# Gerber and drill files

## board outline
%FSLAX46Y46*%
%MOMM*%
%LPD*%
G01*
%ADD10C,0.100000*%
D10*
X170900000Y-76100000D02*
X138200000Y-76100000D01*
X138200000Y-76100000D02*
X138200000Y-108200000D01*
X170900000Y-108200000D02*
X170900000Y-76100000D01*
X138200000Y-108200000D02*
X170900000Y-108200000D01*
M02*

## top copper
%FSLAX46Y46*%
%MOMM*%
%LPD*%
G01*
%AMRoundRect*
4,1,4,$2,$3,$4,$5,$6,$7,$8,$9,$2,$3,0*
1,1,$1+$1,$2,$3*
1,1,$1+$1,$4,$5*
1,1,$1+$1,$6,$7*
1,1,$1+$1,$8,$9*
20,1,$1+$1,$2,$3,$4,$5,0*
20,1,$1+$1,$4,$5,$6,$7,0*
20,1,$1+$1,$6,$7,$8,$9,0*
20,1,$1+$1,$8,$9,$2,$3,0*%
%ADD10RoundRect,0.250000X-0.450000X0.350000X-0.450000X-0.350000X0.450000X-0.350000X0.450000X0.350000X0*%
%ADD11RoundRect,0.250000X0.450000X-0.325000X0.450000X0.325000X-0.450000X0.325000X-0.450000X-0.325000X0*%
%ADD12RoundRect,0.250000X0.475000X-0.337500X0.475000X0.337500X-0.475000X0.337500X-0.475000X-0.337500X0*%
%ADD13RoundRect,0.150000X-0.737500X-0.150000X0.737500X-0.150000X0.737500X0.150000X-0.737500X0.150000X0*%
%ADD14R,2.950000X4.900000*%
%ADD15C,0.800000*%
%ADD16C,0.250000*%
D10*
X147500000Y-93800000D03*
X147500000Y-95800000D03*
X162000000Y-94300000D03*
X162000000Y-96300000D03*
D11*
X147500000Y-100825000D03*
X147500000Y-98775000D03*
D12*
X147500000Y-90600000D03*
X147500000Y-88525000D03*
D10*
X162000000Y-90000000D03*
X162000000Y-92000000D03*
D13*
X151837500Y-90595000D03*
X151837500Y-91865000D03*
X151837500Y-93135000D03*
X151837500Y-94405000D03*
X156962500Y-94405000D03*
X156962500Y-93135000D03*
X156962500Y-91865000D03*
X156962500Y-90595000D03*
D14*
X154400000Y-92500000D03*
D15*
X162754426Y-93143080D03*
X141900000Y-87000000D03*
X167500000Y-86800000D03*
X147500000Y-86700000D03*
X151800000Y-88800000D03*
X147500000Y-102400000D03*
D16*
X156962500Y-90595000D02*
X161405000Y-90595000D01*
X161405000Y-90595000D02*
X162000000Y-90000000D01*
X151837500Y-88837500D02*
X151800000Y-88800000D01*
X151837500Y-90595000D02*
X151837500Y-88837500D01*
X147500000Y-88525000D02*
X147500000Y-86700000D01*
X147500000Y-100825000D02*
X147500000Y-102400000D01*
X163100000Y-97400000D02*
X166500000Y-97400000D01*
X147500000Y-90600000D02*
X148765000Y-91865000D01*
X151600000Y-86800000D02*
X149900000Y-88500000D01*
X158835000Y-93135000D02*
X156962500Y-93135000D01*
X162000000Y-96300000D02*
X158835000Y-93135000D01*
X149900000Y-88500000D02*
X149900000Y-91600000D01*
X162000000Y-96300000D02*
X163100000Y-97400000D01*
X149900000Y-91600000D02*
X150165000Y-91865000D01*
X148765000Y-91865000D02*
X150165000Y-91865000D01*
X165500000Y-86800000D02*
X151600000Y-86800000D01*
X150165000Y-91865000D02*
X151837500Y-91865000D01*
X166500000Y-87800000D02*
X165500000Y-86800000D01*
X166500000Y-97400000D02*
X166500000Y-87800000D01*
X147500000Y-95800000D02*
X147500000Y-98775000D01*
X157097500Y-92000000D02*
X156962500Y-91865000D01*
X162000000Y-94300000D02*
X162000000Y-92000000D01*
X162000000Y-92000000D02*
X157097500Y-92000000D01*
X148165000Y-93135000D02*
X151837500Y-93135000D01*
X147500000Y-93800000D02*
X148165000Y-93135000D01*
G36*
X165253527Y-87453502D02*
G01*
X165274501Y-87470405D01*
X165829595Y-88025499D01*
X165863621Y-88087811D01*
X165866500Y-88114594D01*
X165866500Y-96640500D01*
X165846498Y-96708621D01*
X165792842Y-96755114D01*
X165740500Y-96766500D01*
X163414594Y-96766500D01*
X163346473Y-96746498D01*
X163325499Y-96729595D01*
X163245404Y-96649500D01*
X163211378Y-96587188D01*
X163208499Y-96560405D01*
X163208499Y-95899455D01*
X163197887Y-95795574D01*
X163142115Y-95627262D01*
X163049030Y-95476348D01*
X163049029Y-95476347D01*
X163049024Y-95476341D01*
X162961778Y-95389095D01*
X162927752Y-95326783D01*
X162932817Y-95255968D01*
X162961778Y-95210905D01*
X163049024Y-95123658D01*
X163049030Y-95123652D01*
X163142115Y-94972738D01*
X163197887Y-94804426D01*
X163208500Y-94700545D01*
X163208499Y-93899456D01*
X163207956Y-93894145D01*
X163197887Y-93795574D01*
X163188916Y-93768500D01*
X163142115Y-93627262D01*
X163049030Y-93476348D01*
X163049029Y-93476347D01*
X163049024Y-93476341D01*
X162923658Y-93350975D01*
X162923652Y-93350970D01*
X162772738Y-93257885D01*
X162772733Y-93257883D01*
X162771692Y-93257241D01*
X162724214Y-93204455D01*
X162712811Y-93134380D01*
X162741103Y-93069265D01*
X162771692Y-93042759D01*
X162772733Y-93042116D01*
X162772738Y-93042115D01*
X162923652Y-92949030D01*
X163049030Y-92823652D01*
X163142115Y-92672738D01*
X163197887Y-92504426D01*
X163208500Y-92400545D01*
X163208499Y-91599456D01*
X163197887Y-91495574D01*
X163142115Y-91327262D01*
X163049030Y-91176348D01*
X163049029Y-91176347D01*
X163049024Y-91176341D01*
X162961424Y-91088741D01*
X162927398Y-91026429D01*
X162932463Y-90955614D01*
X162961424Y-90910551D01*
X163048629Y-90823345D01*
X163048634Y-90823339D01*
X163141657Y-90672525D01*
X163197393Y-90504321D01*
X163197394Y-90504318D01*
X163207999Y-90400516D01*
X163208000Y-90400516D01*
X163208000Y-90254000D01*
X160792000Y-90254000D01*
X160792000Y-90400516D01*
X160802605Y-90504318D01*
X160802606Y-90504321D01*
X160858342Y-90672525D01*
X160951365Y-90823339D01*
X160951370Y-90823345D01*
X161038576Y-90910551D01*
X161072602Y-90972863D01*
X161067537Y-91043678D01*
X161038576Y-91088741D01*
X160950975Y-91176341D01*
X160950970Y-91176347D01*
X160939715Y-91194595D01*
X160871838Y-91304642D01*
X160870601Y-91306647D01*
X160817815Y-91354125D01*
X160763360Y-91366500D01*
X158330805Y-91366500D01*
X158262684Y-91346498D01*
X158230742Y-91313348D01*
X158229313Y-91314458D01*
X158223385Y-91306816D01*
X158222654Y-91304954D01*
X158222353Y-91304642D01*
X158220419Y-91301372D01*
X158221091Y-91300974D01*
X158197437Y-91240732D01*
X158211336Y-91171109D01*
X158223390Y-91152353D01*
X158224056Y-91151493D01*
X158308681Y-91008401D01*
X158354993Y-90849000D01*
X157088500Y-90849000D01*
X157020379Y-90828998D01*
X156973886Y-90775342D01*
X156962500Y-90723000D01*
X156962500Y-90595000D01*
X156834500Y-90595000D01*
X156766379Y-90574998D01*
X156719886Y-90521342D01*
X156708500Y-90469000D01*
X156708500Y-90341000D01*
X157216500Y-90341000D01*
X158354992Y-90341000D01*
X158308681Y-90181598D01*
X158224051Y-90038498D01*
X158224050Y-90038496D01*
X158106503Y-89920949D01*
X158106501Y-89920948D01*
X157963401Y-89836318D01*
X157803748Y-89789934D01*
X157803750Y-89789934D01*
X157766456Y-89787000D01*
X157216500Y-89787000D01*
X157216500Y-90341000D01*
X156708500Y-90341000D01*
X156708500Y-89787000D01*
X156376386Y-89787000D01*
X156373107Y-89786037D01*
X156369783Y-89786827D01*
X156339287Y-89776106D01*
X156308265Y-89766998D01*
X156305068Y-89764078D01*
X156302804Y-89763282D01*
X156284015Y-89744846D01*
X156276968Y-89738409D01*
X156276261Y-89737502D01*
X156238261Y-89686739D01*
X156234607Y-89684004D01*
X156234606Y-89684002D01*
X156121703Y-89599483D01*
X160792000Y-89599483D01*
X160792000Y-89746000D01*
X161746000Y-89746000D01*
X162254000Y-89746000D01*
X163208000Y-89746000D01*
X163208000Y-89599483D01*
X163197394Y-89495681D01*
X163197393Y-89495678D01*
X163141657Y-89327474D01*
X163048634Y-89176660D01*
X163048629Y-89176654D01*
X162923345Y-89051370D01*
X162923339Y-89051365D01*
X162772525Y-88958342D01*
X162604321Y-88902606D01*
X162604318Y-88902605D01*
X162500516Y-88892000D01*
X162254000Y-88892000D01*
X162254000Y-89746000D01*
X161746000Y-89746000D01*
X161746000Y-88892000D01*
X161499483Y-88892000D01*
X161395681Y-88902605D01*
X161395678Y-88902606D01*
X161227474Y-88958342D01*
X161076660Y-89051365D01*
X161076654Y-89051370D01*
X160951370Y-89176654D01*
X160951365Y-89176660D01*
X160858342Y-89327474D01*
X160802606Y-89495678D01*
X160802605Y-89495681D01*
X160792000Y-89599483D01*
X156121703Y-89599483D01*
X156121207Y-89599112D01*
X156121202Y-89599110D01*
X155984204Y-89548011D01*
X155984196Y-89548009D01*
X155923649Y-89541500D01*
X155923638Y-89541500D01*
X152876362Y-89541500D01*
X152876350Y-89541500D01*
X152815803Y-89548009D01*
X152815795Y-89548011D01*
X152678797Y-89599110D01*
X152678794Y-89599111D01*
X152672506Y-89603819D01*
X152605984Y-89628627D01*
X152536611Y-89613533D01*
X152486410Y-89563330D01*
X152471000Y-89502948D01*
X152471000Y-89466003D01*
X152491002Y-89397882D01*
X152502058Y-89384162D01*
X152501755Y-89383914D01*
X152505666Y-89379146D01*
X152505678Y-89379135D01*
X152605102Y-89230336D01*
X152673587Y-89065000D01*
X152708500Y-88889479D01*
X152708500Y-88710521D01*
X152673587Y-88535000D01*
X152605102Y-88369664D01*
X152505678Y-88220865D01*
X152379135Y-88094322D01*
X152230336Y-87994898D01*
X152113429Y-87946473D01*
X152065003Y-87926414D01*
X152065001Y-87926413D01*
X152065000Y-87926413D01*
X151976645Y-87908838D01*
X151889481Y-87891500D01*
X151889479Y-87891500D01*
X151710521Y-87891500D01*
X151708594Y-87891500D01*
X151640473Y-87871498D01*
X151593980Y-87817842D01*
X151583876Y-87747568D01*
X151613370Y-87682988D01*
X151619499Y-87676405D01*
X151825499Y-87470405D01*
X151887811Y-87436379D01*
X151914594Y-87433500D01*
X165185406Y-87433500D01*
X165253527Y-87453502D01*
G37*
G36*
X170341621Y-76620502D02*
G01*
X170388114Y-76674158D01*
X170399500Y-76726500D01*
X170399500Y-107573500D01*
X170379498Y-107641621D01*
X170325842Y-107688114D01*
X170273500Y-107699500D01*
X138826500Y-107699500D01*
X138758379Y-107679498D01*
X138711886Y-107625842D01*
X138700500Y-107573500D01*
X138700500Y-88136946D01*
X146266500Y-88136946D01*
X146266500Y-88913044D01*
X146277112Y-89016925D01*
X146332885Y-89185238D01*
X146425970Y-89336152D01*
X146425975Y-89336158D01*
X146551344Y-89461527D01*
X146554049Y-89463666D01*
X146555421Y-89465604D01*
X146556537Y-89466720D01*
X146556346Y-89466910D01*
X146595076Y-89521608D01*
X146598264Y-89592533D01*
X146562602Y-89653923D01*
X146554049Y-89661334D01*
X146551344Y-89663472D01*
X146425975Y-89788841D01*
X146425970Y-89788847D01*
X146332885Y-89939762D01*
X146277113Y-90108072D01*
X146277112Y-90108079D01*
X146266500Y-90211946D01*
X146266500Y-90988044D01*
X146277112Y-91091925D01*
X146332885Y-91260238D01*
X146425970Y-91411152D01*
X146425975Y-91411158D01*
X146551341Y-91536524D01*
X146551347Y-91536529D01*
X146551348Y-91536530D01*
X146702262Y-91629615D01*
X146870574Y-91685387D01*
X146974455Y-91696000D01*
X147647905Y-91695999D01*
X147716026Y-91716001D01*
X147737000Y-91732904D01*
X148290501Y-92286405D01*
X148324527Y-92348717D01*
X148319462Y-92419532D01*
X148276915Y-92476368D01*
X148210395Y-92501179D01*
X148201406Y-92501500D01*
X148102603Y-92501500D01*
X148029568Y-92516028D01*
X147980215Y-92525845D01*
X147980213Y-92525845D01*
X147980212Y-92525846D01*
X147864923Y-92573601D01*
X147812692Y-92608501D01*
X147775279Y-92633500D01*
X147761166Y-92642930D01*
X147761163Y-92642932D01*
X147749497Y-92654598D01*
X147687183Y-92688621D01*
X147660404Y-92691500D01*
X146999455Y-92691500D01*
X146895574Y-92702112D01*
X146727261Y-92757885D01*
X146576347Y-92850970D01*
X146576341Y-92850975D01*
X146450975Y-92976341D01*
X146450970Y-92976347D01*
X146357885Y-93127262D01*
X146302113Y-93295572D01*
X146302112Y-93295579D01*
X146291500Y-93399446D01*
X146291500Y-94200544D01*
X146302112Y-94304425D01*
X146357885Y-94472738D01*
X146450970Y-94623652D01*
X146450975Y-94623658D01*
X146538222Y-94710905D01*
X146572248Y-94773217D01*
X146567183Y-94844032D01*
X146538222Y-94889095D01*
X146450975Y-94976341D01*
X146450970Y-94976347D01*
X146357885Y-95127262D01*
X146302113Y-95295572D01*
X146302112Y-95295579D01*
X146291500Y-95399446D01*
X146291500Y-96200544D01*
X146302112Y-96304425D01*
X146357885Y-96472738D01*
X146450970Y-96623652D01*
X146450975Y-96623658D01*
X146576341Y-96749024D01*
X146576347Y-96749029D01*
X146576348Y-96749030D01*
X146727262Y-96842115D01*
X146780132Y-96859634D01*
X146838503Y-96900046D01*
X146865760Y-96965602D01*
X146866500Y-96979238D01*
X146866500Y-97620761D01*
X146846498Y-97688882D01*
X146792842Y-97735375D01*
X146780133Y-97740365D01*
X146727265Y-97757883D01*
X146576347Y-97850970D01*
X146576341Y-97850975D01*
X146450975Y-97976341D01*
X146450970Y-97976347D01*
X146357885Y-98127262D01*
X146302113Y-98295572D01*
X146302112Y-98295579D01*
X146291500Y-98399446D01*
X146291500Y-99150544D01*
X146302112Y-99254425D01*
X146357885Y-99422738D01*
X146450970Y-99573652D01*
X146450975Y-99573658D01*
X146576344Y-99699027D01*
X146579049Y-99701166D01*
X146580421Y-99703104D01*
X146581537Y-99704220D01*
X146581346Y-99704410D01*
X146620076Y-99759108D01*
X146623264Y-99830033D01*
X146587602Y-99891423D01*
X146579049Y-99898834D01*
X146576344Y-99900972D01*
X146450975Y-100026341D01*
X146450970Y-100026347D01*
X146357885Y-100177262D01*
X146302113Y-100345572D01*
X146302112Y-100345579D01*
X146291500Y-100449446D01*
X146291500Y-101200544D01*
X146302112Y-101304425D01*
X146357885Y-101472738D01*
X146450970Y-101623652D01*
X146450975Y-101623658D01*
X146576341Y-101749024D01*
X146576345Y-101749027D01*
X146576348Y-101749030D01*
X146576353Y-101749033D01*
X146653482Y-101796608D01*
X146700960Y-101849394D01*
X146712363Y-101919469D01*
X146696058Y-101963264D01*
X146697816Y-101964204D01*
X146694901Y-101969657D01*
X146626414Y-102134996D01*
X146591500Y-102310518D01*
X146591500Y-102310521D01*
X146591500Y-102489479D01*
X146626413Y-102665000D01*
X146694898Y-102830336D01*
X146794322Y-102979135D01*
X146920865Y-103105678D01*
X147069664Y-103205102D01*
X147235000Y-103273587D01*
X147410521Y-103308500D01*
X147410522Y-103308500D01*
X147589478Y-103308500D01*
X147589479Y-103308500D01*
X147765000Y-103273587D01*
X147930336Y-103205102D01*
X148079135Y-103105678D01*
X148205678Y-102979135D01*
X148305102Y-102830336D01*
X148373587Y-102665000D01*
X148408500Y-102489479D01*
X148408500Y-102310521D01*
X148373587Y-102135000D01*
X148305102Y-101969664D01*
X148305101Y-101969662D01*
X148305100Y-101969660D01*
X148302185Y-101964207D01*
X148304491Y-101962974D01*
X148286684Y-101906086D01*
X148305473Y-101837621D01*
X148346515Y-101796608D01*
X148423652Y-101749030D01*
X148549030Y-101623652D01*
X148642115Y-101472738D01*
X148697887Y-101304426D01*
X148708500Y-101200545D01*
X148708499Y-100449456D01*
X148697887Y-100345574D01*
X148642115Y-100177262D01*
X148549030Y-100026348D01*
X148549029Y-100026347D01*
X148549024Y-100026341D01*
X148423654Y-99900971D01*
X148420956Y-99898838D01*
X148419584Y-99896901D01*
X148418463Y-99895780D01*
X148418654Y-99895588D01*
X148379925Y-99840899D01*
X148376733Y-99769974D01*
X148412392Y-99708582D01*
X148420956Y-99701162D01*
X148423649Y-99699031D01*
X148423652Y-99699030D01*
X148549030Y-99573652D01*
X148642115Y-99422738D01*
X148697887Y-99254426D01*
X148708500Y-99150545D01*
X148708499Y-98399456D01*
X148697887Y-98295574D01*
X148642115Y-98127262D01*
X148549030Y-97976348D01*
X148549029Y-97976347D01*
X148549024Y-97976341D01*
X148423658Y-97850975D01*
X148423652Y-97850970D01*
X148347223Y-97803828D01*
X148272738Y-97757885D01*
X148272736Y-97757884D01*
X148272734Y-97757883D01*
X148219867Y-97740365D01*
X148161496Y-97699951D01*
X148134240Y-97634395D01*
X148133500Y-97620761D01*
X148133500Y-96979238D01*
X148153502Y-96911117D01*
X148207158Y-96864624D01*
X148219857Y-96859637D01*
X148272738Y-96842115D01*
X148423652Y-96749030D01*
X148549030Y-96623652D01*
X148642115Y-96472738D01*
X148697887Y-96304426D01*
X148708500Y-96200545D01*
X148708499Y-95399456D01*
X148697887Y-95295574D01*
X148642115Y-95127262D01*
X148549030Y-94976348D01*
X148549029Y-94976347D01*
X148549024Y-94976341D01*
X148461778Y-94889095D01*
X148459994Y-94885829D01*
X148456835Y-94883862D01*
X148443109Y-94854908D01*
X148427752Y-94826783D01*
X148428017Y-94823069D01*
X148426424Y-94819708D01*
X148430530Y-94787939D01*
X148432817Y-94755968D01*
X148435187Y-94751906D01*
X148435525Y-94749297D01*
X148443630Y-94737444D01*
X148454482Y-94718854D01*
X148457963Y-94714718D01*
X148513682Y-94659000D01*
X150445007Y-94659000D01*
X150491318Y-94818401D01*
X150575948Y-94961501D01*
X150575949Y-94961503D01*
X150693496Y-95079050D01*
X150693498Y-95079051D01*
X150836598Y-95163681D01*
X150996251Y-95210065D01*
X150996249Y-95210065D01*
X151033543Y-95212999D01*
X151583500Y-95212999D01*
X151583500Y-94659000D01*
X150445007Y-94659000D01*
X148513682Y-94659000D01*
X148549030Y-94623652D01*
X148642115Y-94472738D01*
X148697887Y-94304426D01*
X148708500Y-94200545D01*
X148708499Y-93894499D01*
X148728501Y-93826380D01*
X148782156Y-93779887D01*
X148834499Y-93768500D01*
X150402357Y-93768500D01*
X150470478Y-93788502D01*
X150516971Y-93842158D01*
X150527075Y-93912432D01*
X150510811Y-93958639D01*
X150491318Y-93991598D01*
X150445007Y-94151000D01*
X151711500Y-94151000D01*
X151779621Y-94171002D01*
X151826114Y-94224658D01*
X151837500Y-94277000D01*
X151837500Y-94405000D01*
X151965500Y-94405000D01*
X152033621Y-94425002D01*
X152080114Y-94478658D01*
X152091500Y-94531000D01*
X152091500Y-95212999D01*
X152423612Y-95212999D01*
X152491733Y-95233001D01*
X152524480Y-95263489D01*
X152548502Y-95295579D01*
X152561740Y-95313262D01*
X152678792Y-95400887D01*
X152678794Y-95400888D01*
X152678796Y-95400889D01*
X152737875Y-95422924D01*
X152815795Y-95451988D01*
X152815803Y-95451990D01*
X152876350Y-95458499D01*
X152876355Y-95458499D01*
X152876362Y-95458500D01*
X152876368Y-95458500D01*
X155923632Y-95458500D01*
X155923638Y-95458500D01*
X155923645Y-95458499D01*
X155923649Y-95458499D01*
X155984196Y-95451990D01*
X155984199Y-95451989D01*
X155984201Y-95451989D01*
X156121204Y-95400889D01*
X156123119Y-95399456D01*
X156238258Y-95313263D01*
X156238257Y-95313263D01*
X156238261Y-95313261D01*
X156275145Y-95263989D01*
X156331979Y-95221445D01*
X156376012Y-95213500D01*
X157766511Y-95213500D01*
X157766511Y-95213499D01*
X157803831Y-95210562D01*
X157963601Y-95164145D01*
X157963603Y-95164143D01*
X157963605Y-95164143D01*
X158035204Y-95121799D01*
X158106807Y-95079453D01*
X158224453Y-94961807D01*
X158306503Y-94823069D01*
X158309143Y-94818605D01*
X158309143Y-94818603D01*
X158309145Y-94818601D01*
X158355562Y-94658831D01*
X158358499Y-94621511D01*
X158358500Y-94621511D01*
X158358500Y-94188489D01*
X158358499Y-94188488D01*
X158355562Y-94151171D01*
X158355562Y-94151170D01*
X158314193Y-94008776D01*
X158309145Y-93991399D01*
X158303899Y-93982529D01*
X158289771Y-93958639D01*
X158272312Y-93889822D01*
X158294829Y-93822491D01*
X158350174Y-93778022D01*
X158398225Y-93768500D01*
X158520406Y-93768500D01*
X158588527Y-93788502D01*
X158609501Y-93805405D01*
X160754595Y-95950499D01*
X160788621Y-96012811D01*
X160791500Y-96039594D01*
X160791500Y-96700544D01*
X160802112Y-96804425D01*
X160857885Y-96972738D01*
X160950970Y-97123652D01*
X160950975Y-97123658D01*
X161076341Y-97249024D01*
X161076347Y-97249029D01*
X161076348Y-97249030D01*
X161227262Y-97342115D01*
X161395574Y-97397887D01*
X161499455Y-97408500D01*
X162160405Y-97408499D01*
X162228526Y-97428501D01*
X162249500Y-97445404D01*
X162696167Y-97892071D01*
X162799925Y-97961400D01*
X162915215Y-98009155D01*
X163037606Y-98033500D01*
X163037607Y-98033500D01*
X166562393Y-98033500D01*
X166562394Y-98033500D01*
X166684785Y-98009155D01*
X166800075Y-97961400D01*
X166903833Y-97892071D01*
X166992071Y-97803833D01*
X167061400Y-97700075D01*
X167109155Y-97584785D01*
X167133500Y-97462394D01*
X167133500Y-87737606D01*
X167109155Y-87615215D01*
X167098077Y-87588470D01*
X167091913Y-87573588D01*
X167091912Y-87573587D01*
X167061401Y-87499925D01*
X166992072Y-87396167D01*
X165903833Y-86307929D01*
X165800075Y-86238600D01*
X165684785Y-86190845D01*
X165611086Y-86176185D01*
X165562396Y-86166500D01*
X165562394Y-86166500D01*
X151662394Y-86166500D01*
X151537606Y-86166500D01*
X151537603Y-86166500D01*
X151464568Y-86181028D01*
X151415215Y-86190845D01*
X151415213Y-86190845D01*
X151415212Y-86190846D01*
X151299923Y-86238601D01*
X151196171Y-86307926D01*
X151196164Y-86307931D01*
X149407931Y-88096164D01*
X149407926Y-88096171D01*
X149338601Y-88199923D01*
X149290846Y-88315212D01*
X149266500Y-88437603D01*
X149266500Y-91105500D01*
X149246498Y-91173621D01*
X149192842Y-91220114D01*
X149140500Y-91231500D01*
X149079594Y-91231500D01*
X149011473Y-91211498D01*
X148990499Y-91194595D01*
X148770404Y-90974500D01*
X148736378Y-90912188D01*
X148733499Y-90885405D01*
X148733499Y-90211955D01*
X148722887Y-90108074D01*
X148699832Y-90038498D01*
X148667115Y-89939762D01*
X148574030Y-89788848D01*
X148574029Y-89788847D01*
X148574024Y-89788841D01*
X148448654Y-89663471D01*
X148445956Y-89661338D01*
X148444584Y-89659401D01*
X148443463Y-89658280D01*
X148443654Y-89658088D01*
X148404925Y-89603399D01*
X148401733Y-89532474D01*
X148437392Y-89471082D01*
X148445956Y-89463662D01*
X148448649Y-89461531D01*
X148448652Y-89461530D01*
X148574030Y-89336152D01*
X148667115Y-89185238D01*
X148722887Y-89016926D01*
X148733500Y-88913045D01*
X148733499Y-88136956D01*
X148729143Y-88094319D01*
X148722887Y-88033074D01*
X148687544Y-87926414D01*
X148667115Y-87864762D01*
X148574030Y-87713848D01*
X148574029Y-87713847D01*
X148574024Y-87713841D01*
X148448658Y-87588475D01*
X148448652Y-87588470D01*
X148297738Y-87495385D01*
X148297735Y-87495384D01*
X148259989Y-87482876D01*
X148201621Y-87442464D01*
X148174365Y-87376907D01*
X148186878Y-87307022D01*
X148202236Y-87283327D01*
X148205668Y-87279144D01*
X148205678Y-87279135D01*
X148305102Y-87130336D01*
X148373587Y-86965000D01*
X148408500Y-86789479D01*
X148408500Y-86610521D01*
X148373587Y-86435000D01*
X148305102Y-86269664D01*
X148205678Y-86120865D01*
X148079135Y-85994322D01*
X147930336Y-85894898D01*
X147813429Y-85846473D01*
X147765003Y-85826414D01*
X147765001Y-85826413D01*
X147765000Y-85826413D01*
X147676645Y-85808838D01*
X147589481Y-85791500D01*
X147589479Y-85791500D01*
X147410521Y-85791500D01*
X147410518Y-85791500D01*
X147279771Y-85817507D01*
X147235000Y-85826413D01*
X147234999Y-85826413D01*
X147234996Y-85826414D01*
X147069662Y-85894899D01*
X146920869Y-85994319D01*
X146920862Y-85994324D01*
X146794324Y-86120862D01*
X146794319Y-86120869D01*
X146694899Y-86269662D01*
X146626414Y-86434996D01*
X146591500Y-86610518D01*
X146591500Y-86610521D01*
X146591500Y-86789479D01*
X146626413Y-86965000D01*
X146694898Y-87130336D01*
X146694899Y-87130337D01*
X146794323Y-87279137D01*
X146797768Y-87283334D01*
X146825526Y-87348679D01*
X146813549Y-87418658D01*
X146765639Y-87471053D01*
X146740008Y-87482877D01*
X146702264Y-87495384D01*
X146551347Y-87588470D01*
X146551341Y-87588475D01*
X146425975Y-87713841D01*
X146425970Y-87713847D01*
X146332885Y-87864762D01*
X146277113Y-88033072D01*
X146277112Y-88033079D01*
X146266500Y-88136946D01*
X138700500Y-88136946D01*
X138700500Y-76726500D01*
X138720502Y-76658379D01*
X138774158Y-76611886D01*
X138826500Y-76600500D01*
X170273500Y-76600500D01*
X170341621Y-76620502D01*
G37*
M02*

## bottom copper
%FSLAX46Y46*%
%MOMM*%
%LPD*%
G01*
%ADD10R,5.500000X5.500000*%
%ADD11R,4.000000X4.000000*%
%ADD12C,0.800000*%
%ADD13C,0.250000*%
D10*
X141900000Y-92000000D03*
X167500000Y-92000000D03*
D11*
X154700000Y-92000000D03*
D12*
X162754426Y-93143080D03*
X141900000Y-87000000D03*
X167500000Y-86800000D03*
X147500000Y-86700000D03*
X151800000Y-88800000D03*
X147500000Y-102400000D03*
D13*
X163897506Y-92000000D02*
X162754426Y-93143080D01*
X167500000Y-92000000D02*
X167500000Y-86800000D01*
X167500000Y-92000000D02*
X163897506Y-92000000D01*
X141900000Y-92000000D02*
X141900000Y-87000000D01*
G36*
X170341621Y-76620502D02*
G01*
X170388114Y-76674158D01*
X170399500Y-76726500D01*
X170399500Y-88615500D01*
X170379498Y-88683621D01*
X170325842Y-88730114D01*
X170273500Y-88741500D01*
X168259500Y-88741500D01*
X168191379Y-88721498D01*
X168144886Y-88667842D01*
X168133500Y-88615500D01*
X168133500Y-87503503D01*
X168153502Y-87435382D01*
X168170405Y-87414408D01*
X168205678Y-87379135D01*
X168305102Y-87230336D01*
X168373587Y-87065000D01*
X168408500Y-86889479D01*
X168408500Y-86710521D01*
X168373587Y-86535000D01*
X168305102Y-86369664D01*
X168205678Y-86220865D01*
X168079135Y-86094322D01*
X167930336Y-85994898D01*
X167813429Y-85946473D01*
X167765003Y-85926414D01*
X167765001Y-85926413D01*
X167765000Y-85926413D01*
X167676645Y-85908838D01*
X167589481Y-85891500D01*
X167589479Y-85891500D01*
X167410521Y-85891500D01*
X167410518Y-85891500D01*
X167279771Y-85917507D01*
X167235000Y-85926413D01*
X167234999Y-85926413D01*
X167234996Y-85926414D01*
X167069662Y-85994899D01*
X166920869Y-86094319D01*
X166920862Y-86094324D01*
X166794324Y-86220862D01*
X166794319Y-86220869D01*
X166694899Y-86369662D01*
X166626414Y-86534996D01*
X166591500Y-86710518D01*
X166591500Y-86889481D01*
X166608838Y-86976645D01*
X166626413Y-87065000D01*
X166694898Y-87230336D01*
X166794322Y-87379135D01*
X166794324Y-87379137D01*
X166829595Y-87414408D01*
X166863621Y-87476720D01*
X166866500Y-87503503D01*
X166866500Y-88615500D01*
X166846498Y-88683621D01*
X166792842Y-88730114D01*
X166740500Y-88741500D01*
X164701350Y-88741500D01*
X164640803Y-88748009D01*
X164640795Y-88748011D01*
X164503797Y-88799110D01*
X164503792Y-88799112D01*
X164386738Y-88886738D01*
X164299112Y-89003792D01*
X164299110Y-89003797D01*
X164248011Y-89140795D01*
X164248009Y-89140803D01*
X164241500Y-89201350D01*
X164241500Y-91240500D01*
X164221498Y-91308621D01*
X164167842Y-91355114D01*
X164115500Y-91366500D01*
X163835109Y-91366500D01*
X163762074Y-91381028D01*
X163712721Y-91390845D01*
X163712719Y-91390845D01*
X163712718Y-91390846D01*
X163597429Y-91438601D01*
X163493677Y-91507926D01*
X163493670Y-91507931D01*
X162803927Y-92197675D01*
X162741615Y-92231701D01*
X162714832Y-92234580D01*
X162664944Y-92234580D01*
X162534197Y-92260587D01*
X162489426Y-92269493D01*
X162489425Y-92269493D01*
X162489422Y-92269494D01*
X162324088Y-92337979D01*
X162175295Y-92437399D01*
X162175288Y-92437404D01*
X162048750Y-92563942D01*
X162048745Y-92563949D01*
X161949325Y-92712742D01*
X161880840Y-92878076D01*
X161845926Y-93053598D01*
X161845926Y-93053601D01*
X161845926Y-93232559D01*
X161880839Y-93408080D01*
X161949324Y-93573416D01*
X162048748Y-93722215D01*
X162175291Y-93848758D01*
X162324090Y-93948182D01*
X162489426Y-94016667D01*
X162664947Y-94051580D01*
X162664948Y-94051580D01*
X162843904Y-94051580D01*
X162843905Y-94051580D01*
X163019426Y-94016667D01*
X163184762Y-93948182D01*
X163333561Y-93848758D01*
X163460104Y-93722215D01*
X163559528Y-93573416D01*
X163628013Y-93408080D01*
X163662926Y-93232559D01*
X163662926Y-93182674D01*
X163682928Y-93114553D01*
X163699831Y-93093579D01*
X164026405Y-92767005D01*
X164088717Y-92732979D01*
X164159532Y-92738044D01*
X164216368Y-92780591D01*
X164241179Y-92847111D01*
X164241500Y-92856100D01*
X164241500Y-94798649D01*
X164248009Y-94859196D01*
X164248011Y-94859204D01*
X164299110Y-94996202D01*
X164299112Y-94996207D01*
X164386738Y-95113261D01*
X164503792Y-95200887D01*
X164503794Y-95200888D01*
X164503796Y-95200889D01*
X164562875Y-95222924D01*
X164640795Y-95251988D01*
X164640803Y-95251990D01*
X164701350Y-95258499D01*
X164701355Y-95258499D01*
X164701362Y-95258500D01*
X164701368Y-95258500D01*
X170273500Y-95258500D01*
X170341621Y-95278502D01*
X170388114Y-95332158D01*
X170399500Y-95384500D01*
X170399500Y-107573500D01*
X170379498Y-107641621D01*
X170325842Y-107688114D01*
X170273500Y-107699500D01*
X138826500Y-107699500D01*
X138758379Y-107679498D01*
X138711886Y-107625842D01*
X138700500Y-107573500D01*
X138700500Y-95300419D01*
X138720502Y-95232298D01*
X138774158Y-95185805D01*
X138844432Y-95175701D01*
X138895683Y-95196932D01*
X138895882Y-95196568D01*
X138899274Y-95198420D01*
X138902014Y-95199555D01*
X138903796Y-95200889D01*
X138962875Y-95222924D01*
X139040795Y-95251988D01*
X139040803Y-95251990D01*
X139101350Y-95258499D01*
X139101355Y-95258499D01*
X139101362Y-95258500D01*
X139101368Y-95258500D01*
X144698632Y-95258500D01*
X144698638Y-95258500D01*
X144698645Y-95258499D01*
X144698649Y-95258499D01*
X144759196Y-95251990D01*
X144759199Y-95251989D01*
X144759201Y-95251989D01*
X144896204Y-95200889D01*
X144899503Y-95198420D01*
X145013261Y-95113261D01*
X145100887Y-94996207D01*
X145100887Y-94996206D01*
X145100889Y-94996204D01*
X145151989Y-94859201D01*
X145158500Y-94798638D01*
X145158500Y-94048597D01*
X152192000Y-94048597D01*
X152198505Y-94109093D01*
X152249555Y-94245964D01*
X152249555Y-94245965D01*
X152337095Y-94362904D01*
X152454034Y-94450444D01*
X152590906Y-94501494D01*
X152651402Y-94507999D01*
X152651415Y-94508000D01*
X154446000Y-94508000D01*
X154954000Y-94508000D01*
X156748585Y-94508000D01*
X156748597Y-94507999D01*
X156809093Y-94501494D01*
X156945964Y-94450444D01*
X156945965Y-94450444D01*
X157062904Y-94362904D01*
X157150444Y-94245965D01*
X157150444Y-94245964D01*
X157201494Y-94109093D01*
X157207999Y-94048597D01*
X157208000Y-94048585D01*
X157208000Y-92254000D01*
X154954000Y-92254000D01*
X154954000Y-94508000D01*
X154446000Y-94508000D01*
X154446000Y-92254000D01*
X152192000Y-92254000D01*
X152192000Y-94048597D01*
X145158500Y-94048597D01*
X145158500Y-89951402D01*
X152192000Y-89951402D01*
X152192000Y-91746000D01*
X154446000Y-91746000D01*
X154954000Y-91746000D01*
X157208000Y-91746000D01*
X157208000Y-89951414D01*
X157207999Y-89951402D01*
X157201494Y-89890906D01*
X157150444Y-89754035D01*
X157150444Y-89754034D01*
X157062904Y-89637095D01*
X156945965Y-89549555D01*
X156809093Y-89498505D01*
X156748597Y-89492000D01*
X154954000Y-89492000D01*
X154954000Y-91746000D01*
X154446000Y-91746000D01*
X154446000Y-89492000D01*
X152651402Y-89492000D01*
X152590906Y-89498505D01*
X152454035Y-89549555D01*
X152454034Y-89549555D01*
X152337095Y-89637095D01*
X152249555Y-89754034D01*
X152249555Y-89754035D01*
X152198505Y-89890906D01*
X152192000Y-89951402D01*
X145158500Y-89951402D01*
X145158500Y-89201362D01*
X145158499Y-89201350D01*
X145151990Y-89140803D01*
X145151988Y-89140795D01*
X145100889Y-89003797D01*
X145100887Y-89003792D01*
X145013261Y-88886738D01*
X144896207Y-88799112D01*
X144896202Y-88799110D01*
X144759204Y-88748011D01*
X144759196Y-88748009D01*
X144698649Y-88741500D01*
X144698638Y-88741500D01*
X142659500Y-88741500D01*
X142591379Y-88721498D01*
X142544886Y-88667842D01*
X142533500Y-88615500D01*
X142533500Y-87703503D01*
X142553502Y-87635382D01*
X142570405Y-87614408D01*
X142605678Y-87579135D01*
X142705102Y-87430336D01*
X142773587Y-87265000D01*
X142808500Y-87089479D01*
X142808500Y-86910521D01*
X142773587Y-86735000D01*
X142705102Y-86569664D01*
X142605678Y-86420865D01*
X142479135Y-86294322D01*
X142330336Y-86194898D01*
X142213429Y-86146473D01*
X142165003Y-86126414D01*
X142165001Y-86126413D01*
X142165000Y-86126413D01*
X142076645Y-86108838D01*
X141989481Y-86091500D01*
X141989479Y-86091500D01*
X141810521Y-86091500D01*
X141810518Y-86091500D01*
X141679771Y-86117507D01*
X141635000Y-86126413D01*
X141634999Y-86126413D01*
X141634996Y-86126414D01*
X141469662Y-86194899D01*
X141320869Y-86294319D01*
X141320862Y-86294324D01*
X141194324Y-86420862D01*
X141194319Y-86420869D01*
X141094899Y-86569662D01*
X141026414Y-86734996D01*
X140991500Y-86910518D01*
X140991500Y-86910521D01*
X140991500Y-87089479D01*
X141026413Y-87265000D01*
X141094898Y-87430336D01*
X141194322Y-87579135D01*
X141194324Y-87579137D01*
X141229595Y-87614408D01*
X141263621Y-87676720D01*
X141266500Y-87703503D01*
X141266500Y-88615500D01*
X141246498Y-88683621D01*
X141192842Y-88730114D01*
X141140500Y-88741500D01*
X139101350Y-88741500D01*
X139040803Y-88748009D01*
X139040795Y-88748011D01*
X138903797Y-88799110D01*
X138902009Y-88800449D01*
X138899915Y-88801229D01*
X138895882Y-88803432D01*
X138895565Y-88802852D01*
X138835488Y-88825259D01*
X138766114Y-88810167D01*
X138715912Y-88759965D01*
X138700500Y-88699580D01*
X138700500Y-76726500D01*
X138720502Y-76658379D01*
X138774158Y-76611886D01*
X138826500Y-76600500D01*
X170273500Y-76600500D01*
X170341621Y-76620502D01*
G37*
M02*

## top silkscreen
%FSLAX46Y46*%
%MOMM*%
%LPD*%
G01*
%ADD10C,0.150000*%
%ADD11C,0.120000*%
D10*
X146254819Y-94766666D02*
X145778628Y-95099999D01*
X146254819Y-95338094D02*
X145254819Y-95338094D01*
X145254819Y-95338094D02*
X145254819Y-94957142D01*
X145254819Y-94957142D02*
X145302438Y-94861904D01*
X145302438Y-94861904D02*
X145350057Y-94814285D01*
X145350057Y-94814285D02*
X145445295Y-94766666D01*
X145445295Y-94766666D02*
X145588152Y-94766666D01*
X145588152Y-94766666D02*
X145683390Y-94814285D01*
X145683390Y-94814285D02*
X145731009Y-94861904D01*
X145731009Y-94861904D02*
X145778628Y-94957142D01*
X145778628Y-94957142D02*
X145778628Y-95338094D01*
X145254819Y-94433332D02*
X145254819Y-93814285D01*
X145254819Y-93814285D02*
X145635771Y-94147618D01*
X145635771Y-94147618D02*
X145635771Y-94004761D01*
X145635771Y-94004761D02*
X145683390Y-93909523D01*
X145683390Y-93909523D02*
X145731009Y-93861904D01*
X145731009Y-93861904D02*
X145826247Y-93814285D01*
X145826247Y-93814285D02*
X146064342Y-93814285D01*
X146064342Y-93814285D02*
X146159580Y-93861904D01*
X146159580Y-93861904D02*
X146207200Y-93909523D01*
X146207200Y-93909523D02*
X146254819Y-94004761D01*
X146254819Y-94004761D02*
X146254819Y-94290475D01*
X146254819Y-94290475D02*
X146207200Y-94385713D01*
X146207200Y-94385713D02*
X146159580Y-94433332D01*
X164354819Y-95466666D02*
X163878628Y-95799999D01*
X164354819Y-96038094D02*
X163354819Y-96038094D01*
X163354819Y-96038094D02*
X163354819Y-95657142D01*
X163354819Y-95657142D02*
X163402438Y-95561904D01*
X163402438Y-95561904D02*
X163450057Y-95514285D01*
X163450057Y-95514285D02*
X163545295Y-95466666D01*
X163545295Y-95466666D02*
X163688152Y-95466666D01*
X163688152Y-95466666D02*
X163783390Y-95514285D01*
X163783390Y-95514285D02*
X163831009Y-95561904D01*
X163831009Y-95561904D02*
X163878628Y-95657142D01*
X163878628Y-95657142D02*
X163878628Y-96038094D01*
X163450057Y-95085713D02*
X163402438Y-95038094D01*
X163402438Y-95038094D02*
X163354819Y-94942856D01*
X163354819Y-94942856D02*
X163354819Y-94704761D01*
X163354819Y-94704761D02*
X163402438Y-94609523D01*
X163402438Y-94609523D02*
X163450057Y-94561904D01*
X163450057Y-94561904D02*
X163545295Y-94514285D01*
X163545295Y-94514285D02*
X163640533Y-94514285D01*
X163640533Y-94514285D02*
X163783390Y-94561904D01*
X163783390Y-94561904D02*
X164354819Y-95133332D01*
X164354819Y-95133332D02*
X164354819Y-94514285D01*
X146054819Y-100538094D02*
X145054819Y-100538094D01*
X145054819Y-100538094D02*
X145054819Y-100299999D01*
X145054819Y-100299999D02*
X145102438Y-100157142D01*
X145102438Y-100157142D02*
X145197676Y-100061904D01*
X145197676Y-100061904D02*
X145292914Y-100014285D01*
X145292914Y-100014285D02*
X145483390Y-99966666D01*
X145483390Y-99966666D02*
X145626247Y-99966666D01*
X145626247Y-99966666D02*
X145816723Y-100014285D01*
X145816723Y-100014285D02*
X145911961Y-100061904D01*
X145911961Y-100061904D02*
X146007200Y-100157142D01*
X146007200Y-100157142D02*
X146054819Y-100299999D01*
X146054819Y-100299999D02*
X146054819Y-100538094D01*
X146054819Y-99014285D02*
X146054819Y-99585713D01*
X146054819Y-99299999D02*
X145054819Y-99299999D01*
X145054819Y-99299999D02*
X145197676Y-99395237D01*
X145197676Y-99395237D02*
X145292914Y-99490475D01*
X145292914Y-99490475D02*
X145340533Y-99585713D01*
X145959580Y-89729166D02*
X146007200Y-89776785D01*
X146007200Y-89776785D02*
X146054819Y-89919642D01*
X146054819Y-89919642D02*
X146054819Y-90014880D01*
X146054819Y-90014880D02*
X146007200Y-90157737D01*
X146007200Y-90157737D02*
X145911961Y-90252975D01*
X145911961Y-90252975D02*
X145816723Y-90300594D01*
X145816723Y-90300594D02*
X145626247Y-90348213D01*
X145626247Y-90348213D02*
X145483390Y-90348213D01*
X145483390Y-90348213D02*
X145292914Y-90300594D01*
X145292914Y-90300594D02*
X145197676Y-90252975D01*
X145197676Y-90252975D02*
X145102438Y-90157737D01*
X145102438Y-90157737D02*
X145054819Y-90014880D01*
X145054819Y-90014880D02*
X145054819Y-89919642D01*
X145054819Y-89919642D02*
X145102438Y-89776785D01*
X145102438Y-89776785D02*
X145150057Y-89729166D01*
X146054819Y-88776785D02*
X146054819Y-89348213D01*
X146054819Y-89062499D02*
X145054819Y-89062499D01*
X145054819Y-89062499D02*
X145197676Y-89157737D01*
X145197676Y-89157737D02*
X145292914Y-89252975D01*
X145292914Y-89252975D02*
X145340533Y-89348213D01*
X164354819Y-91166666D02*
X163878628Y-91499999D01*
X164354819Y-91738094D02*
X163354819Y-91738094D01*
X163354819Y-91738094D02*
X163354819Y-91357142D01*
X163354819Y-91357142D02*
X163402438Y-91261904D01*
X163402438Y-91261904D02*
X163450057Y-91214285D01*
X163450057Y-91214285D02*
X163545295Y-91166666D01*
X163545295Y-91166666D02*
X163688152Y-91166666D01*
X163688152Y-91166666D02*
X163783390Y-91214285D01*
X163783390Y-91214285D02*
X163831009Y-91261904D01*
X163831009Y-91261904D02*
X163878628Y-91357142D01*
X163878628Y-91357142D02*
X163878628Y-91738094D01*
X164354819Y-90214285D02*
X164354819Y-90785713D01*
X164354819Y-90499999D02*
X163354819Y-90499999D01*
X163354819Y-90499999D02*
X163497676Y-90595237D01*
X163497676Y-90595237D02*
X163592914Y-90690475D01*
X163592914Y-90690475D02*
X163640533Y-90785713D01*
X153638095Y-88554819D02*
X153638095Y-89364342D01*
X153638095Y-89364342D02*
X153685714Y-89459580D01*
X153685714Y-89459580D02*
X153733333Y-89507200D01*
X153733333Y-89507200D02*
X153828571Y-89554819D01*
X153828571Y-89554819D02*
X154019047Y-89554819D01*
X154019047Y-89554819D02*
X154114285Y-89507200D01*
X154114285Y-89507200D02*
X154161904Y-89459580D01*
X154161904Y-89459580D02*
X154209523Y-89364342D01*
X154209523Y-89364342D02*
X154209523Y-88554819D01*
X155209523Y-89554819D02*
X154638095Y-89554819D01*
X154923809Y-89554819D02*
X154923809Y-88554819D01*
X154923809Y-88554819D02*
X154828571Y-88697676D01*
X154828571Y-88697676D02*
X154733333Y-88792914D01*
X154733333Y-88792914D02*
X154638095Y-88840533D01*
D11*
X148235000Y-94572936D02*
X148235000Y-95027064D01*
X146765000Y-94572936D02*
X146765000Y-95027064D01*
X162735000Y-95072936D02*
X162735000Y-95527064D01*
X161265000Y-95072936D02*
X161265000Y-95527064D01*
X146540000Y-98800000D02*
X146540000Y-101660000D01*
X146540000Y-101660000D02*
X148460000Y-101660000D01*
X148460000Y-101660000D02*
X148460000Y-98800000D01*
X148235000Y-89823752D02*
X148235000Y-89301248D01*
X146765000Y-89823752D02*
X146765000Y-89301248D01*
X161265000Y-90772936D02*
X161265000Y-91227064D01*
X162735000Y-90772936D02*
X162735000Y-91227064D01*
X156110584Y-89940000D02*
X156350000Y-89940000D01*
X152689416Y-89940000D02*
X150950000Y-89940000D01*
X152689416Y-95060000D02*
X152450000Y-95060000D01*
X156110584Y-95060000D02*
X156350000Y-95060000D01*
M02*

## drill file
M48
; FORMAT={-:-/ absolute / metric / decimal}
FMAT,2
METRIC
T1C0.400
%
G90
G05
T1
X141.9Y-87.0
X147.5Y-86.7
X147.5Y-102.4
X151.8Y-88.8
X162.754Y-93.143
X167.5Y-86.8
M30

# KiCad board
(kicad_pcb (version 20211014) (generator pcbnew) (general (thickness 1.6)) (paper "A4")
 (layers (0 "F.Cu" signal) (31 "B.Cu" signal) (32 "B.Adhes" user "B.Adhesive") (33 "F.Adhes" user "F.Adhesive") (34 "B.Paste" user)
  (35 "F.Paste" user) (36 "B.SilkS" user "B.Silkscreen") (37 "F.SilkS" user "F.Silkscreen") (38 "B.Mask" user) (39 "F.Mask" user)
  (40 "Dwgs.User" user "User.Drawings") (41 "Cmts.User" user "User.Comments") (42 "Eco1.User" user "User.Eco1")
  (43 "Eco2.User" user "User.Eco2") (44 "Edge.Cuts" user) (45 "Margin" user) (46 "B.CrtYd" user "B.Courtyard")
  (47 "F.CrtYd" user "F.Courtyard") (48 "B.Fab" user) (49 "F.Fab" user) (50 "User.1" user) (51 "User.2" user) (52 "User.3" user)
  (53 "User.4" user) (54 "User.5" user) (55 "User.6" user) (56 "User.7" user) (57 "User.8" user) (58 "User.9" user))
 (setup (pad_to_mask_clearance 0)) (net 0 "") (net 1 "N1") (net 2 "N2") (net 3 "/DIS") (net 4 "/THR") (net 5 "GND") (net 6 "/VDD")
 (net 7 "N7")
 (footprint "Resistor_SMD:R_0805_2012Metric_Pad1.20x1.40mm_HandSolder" (layer "F.Cu") (at 147.5 94.8 -90)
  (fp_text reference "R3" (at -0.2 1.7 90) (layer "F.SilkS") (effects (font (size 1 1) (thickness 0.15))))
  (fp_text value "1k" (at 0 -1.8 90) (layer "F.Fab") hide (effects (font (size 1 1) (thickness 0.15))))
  (fp_line (start -0.227064 -0.735) (end 0.227064 -0.735) (layer "F.SilkS") (width 0.12))
  (fp_line (start -0.227064 0.735) (end 0.227064 0.735) (layer "F.SilkS") (width 0.12))
  (pad "1" smd roundrect (at -1 0 270) (size 1.2 1.4) (layers "F.Cu" "F.Paste" "F.Mask") (roundrect_rratio 0.208333) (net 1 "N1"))
  (pad "2" smd roundrect (at 1 0 270) (size 1.2 1.4) (layers "F.Cu" "F.Paste" "F.Mask") (roundrect_rratio 0.208333) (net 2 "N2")))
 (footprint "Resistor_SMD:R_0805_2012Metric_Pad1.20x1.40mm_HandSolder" (layer "F.Cu") (at 162 95.3 -90)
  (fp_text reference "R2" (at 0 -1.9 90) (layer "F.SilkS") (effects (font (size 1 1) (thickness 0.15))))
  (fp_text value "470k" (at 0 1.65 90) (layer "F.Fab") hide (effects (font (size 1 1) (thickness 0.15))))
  (fp_line (start -0.227064 -0.735) (end 0.227064 -0.735) (layer "F.SilkS") (width 0.12))
  (fp_line (start -0.227064 0.735) (end 0.227064 0.735) (layer "F.SilkS") (width 0.12))
  (pad "1" smd roundrect (at -1 0 270) (size 1.2 1.4) (layers "F.Cu" "F.Paste" "F.Mask") (roundrect_rratio 0.208333) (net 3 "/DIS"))
  (pad "2" smd roundrect (at 1 0 270) (size 1.2 1.4) (layers "F.Cu" "F.Paste" "F.Mask") (roundrect_rratio 0.208333) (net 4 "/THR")))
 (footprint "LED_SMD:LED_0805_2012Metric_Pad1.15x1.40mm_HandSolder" (layer "F.Cu") (at 147.5 99.8 90)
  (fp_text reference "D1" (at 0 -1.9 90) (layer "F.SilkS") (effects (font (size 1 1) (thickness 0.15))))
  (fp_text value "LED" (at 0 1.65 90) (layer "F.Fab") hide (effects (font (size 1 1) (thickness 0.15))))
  (fp_line (start 1 -0.96) (end -1.86 -0.96) (layer "F.SilkS") (width 0.12))
  (fp_line (start -1.86 -0.96) (end -1.86 0.96) (layer "F.SilkS") (width 0.12))
  (fp_line (start -1.86 0.96) (end 1 0.96) (layer "F.SilkS") (width 0.12))
  (pad "1" smd roundrect (at -1.025 0 90) (size 1.15 1.4) (layers "F.Cu" "F.Paste" "F.Mask") (roundrect_rratio 0.217391) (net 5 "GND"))
  (pad "2" smd roundrect (at 1.025 0 90) (size 1.15 1.4) (layers "F.Cu" "F.Paste" "F.Mask") (roundrect_rratio 0.217391) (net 2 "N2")))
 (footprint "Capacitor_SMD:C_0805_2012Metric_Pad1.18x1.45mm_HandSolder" (layer "F.Cu") (at 147.5 89.5625 90)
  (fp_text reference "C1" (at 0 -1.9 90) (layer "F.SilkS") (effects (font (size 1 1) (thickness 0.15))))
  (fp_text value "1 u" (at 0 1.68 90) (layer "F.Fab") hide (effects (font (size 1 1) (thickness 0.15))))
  (fp_line (start -0.261252 0.735) (end 0.261252 0.735) (layer "F.SilkS") (width 0.12))
  (fp_line (start -0.261252 -0.735) (end 0.261252 -0.735) (layer "F.SilkS") (width 0.12))
  (pad "1" smd roundrect (at -1.0375 0 90) (size 1.175 1.45) (layers "F.Cu" "F.Paste" "F.Mask") (roundrect_rratio 0.212766) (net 4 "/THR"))
  (pad "2" smd roundrect (at 1.0375 0 90) (size 1.175 1.45) (layers "F.Cu" "F.Paste" "F.Mask") (roundrect_rratio 0.212766) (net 5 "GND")))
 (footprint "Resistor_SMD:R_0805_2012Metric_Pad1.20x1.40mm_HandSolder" (layer "F.Cu") (at 162 91 -90)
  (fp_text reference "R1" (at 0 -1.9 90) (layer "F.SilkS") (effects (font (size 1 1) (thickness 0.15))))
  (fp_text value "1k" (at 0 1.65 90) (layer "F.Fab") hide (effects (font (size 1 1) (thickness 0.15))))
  (fp_line (start -0.227064 0.735) (end 0.227064 0.735) (layer "F.SilkS") (width 0.12))
  (fp_line (start -0.227064 -0.735) (end 0.227064 -0.735) (layer "F.SilkS") (width 0.12))
  (pad "1" smd roundrect (at -1 0 270) (size 1.2 1.4) (layers "F.Cu" "F.Paste" "F.Mask") (roundrect_rratio 0.208333) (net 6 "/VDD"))
  (pad "2" smd roundrect (at 1 0 270) (size 1.2 1.4) (layers "F.Cu" "F.Paste" "F.Mask") (roundrect_rratio 0.208333) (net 3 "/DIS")))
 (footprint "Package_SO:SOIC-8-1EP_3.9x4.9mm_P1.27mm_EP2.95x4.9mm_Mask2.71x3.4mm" (layer "F.Cu") (at 154.4 92.5)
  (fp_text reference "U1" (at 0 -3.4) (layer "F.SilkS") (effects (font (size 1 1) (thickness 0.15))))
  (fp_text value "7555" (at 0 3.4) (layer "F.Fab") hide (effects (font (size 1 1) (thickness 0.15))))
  (fp_line (start 1.710584 -2.56) (end 1.95 -2.56) (layer "F.SilkS") (width 0.12))
  (fp_line (start -1.710584 -2.56) (end -3.45 -2.56) (layer "F.SilkS") (width 0.12))
  (fp_line (start -1.710584 2.56) (end -1.95 2.56) (layer "F.SilkS") (width 0.12))
  (fp_line (start 1.710584 2.56) (end 1.95 2.56) (layer "F.SilkS") (width 0.12))
  (pad "" smd roundrect (at -0.68 0.85) (size 1.09 1.37) (layers "F.Paste") (roundrect_rratio 0.229358))
  (pad "" smd roundrect (at 0.68 -0.85) (size 1.09 1.37) (layers "F.Paste") (roundrect_rratio 0.229358))
  (pad "" smd roundrect (at -0.68 -0.85) (size 1.09 1.37) (layers "F.Paste") (roundrect_rratio 0.229358))
  (pad "" smd roundrect (at 0.68 0.85) (size 1.09 1.37) (layers "F.Paste") (roundrect_rratio 0.229358))
  (pad "" smd rect (at 0 0) (size 2.71 3.4) (layers "F.Mask"))
  (pad "1" smd roundrect (at -2.5625 -1.905) (size 1.775 0.6) (layers "F.Cu" "F.Paste" "F.Mask") (roundrect_rratio 0.25) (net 5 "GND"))
  (pad "2" smd roundrect (at -2.5625 -0.635) (size 1.775 0.6) (layers "F.Cu" "F.Paste" "F.Mask") (roundrect_rratio 0.25) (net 4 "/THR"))
  (pad "3" smd roundrect (at -2.5625 0.635) (size 1.775 0.6) (layers "F.Cu" "F.Paste" "F.Mask") (roundrect_rratio 0.25) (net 1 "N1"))
  (pad "4" smd roundrect (at -2.5625 1.905) (size 1.775 0.6) (layers "F.Cu" "F.Paste" "F.Mask") (roundrect_rratio 0.25) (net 6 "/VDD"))
  (pad "5" smd roundrect (at 2.5625 1.905) (size 1.775 0.6) (layers "F.Cu" "F.Paste" "F.Mask") (roundrect_rratio 0.25) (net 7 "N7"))
  (pad "6" smd roundrect (at 2.5625 0.635) (size 1.775 0.6) (layers "F.Cu" "F.Paste" "F.Mask") (roundrect_rratio 0.25) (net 4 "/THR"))
  (pad "7" smd roundrect (at 2.5625 -0.635) (size 1.775 0.6) (layers "F.Cu" "F.Paste" "F.Mask") (roundrect_rratio 0.25) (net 3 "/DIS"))
  (pad "8" smd roundrect (at 2.5625 -1.905) (size 1.775 0.6) (layers "F.Cu" "F.Paste" "F.Mask") (roundrect_rratio 0.25) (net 6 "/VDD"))
  (pad "9" smd rect (at 0 0) (size 2.95 4.9) (layers "F.Cu")))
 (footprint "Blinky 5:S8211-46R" (layer "B.Cu") (at 154.7 92)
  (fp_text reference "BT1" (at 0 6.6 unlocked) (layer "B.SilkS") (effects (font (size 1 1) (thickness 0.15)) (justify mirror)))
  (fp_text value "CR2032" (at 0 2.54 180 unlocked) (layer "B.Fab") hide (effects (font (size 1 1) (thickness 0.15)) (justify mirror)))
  (pad "1" smd rect (at -12.8 0) (size 5.5 5.5) (layers "B.Cu" "B.Paste" "B.Mask") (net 6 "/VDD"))
  (pad "1" smd rect (at 12.8 0) (size 5.5 5.5) (layers "B.Cu" "B.Paste" "B.Mask") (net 6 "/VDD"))
  (pad "2" smd rect (at 0 0) (size 4 4) (layers "B.Cu" "B.Paste" "B.Mask") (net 5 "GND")))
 (gr_line (start 170.9 76.1) (end 138.2 76.1) (layer "Edge.Cuts") (width 0.1))
 (gr_line (start 138.2 76.1) (end 138.2 108.2) (layer "Edge.Cuts") (width 0.1))
 (gr_line (start 170.9 108.2) (end 170.9 76.1) (layer "Edge.Cuts") (width 0.1))
 (gr_line (start 138.2 108.2) (end 170.9 108.2) (layer "Edge.Cuts") (width 0.1))
 (segment (start 156.9625 90.595) (end 161.405 90.595) (width 0.25) (layer "F.Cu") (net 6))
 (segment (start 161.405 90.595) (end 162 90) (width 0.25) (layer "F.Cu") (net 6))
 (via (at 162.754426 93.14308) (size 0.8) (drill 0.4) (layers "F.Cu" "B.Cu") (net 6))
 (via (at 141.9 87) (size 0.8) (drill 0.4) (layers "F.Cu" "B.Cu") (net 6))
 (via (at 167.5 86.8) (size 0.8) (drill 0.4) (layers "F.Cu" "B.Cu") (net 6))
 (segment (start 163.897506 92) (end 162.754426 93.14308) (width 0.25) (layer "B.Cu") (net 6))
 (segment (start 167.5 92) (end 167.5 86.8) (width 0.25) (layer "B.Cu") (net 6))
 (segment (start 167.5 92) (end 163.897506 92) (width 0.25) (layer "B.Cu") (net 6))
 (segment (start 141.9 92) (end 141.9 87) (width 0.25) (layer "B.Cu") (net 6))
 (segment (start 151.8375 88.8375) (end 151.8 88.8) (width 0.25) (layer "F.Cu") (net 5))
 (segment (start 151.8375 90.595) (end 151.8375 88.8375) (width 0.25) (layer "F.Cu") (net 5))
 (segment (start 147.5 88.525) (end 147.5 86.7) (width 0.25) (layer "F.Cu") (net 5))
 (segment (start 147.5 100.825) (end 147.5 102.4) (width 0.25) (layer "F.Cu") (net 5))
 (via (at 147.5 86.7) (size 0.8) (drill 0.4) (layers "F.Cu" "B.Cu") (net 5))
 (via (at 151.8 88.8) (size 0.8) (drill 0.4) (layers "F.Cu" "B.Cu") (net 5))
 (via (at 147.5 102.4) (size 0.8) (drill 0.4) (layers "F.Cu" "B.Cu") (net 5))
 (segment (start 163.1 97.4) (end 166.5 97.4) (width 0.25) (layer "F.Cu") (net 4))
 (segment (start 147.5 90.6) (end 148.765 91.865) (width 0.25) (layer "F.Cu") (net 4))
 (segment (start 151.6 86.8) (end 149.9 88.5) (width 0.25) (layer "F.Cu") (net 4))
 (segment (start 158.835 93.135) (end 156.9625 93.135) (width 0.25) (layer "F.Cu") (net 4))
 (segment (start 162 96.3) (end 158.835 93.135) (width 0.25) (layer "F.Cu") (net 4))
 (segment (start 149.9 88.5) (end 149.9 91.6) (width 0.25) (layer "F.Cu") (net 4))
 (segment (start 162 96.3) (end 163.1 97.4) (width 0.25) (layer "F.Cu") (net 4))
 (segment (start 149.9 91.6) (end 150.165 91.865) (width 0.25) (layer "F.Cu") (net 4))
 (segment (start 148.765 91.865) (end 150.165 91.865) (width 0.25) (layer "F.Cu") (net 4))
 (segment (start 165.5 86.8) (end 151.6 86.8) (width 0.25) (layer "F.Cu") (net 4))
 (segment (start 150.165 91.865) (end 151.8375 91.865) (width 0.25) (layer "F.Cu") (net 4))
 (segment (start 166.5 87.8) (end 165.5 86.8) (width 0.25) (layer "F.Cu") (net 4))
 (segment (start 166.5 97.4) (end 166.5 87.8) (width 0.25) (layer "F.Cu") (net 4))
 (segment (start 147.5 95.8) (end 147.5 98.775) (width 0.25) (layer "F.Cu") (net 2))
 (segment (start 157.0975 92) (end 156.9625 91.865) (width 0.25) (layer "F.Cu") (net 3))
 (segment (start 162 94.3) (end 162 92) (width 0.25) (layer "F.Cu") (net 3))
 (segment (start 162 92) (end 157.0975 92) (width 0.25) (layer "F.Cu") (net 3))
 (segment (start 148.165 93.135) (end 151.8375 93.135) (width 0.25) (layer "F.Cu") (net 1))
 (segment (start 147.5 93.8) (end 148.165 93.135) (width 0.25) (layer "F.Cu") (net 1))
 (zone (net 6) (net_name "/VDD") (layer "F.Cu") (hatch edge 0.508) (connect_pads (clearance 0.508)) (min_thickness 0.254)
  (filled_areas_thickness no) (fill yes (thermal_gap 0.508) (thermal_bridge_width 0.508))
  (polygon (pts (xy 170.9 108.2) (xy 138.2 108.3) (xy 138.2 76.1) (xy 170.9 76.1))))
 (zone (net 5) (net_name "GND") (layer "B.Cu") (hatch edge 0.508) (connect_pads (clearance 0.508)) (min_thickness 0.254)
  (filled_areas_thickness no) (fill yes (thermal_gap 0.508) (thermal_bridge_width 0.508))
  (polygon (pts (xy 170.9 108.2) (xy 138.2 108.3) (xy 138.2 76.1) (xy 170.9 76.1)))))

